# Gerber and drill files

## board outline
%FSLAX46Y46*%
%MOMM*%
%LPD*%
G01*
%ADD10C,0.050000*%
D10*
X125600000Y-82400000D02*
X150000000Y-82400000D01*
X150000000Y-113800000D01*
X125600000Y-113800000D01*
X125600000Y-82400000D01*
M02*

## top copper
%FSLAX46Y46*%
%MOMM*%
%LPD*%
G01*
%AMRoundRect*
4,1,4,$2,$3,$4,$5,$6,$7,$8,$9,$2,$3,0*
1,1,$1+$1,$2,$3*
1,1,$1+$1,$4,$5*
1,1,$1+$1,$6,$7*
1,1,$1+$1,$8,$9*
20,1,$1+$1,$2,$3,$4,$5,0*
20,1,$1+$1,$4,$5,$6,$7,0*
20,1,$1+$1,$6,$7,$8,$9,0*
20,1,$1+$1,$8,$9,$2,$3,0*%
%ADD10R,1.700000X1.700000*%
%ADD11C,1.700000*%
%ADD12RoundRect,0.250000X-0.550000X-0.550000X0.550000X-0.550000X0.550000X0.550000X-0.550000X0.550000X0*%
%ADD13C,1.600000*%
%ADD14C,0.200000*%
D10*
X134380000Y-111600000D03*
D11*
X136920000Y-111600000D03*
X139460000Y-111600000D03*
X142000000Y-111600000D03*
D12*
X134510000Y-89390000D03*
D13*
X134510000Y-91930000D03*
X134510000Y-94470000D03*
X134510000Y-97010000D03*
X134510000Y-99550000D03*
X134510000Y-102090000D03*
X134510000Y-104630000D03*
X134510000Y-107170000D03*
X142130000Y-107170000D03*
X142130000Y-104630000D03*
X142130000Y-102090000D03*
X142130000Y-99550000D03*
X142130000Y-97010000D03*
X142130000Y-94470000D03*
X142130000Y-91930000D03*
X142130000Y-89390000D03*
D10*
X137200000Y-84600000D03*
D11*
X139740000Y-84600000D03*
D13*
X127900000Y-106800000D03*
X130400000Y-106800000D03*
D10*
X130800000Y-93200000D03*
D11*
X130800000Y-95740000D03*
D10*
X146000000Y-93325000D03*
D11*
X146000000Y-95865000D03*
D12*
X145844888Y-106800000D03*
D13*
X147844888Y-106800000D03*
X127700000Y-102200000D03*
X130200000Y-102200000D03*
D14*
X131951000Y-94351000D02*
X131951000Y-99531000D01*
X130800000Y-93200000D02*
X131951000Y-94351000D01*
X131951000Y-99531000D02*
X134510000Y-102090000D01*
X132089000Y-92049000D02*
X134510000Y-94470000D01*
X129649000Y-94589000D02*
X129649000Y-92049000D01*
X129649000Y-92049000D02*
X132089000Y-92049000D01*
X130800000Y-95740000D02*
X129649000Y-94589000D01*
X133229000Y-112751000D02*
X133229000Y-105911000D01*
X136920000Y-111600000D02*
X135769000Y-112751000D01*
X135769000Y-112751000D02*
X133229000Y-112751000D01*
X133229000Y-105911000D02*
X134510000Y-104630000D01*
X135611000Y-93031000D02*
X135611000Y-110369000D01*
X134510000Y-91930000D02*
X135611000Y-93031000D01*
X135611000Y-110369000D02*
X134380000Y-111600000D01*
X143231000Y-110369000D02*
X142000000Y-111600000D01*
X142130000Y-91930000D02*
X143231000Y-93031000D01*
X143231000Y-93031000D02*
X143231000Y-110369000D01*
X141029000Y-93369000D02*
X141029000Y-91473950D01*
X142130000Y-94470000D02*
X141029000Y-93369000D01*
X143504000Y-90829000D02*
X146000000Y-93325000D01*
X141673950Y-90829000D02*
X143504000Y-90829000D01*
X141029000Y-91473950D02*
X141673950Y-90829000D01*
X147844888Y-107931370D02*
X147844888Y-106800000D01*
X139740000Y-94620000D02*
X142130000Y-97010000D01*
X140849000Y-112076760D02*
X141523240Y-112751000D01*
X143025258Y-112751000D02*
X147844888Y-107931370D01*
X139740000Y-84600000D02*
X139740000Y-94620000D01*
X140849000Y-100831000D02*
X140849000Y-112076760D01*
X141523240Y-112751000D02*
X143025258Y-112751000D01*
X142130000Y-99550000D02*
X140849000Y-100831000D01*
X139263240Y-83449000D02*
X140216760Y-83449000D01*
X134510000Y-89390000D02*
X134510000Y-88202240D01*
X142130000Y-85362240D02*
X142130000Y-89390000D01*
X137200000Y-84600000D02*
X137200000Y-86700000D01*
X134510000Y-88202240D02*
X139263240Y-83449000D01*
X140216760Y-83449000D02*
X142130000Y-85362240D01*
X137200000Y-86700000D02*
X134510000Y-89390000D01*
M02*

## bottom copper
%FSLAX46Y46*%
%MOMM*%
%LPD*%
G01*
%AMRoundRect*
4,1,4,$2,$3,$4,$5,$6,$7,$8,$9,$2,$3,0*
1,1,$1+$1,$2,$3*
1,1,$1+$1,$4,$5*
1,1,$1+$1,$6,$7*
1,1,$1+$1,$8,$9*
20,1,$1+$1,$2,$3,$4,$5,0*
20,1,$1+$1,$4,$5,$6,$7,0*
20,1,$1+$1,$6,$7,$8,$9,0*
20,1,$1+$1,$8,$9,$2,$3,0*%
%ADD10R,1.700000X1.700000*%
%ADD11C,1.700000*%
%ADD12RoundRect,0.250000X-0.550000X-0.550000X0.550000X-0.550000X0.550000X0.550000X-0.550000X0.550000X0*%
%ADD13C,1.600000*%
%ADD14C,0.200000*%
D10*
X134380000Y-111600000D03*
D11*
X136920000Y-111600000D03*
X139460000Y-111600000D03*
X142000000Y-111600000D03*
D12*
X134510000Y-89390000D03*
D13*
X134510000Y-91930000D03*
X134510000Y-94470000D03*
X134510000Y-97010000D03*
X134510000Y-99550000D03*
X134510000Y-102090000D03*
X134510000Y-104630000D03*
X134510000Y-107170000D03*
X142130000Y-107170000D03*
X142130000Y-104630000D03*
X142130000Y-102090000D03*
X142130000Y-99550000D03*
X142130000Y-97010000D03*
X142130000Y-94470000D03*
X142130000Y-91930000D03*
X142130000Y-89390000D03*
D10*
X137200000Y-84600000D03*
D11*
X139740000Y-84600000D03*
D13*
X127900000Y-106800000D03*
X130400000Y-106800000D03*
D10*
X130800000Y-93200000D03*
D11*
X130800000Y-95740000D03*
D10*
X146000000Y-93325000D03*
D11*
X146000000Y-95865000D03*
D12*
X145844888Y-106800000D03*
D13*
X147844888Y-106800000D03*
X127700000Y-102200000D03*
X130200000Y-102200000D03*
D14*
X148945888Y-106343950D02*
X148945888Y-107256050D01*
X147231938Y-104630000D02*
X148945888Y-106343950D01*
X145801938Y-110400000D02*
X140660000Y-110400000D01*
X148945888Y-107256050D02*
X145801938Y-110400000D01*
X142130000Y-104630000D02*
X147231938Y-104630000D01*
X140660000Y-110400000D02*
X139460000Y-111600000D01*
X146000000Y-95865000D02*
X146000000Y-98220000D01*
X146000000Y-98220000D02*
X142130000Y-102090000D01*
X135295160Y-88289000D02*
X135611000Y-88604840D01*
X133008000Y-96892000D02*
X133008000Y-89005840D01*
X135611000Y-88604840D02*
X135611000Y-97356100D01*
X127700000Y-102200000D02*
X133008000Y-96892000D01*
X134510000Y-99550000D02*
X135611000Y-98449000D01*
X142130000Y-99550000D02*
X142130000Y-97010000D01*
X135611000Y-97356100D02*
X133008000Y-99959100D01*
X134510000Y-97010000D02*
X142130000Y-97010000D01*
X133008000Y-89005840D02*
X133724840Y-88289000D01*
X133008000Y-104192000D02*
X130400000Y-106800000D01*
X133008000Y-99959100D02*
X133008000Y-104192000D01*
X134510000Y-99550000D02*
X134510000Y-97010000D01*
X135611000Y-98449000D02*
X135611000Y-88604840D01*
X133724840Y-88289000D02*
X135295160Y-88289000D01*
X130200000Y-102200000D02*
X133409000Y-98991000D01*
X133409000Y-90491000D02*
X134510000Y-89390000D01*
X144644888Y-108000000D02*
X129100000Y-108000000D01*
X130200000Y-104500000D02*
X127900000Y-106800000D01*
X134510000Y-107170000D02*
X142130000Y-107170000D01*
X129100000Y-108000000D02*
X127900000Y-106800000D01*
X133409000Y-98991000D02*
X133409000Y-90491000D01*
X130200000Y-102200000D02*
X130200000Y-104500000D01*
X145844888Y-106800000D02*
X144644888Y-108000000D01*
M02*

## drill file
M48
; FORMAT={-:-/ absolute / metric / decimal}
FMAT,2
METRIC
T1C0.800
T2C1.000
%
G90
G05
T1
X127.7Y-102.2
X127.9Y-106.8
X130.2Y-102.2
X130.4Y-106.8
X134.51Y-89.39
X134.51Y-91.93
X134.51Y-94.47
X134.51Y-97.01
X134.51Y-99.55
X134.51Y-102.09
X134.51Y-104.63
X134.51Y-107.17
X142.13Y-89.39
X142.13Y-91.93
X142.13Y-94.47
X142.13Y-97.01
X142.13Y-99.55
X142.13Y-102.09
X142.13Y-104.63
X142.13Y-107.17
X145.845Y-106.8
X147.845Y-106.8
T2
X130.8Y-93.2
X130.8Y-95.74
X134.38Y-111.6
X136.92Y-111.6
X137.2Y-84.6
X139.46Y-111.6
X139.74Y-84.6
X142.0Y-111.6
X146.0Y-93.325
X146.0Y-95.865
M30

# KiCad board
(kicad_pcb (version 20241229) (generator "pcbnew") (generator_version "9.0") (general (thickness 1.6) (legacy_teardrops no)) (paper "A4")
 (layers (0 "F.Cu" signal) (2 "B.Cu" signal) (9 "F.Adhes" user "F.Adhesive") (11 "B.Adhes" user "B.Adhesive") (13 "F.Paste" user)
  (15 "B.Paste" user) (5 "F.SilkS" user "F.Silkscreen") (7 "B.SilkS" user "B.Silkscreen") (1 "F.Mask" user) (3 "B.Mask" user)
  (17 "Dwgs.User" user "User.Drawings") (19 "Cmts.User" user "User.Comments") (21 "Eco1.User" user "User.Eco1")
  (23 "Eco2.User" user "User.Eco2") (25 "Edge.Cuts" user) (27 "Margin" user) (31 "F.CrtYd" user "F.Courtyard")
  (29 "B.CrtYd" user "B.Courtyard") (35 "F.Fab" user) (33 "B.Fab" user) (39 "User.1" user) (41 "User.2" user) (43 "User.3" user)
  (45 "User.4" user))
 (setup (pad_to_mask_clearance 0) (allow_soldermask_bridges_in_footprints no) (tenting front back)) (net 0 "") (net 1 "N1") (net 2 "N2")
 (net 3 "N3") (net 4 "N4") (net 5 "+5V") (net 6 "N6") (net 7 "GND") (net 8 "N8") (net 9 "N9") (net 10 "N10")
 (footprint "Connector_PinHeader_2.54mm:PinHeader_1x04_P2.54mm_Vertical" (layer "F.Cu") (at 134.38 111.6 90)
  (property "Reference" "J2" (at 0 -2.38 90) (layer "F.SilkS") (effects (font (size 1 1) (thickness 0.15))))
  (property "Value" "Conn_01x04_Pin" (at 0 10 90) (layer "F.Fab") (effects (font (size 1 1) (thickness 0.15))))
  (pad "1" thru_hole rect (at 0 0 90) (size 1.7 1.7) (drill 1) (layers "*.Cu" "*.Mask") (remove_unused_layers no) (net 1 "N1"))
  (pad "2" thru_hole circle (at 0 2.54 90) (size 1.7 1.7) (drill 1) (layers "*.Cu" "*.Mask") (remove_unused_layers no) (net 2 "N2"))
  (pad "3" thru_hole circle (at 0 5.08 90) (size 1.7 1.7) (drill 1) (layers "*.Cu" "*.Mask") (remove_unused_layers no) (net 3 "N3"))
  (pad "4" thru_hole circle (at 0 7.62 90) (size 1.7 1.7) (drill 1) (layers "*.Cu" "*.Mask") (remove_unused_layers no) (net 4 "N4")))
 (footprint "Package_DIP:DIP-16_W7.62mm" (layer "F.Cu") (at 134.51 89.39)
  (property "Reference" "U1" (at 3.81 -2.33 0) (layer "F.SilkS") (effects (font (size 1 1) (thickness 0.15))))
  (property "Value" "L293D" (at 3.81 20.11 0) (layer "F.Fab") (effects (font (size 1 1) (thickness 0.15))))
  (pad "1" thru_hole roundrect (at 0 0) (size 1.6 1.6) (drill 0.8) (layers "*.Cu" "*.Mask") (remove_unused_layers no)
   (roundrect_rratio 0.15625) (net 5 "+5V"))
  (pad "2" thru_hole circle (at 0 2.54) (size 1.6 1.6) (drill 0.8) (layers "*.Cu" "*.Mask") (remove_unused_layers no) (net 1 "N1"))
  (pad "3" thru_hole circle (at 0 5.08) (size 1.6 1.6) (drill 0.8) (layers "*.Cu" "*.Mask") (remove_unused_layers no) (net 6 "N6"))
  (pad "4" thru_hole circle (at 0 7.62) (size 1.6 1.6) (drill 0.8) (layers "*.Cu" "*.Mask") (remove_unused_layers no) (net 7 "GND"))
  (pad "5" thru_hole circle (at 0 10.16) (size 1.6 1.6) (drill 0.8) (layers "*.Cu" "*.Mask") (remove_unused_layers no) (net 7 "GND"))
  (pad "6" thru_hole circle (at 0 12.7) (size 1.6 1.6) (drill 0.8) (layers "*.Cu" "*.Mask") (remove_unused_layers no) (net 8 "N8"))
  (pad "7" thru_hole circle (at 0 15.24) (size 1.6 1.6) (drill 0.8) (layers "*.Cu" "*.Mask") (remove_unused_layers no) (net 2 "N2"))
  (pad "8" thru_hole circle (at 0 17.78) (size 1.6 1.6) (drill 0.8) (layers "*.Cu" "*.Mask") (remove_unused_layers no) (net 5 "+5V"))
  (pad "9" thru_hole circle (at 7.62 17.78) (size 1.6 1.6) (drill 0.8) (layers "*.Cu" "*.Mask") (remove_unused_layers no) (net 5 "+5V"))
  (pad "10" thru_hole circle (at 7.62 15.24) (size 1.6 1.6) (drill 0.8) (layers "*.Cu" "*.Mask") (remove_unused_layers no) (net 3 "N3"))
  (pad "11" thru_hole circle (at 7.62 12.7) (size 1.6 1.6) (drill 0.8) (layers "*.Cu" "*.Mask") (remove_unused_layers no) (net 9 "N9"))
  (pad "12" thru_hole circle (at 7.62 10.16) (size 1.6 1.6) (drill 0.8) (layers "*.Cu" "*.Mask") (remove_unused_layers no) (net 7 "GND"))
  (pad "13" thru_hole circle (at 7.62 7.62) (size 1.6 1.6) (drill 0.8) (layers "*.Cu" "*.Mask") (remove_unused_layers no) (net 7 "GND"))
  (pad "14" thru_hole circle (at 7.62 5.08) (size 1.6 1.6) (drill 0.8) (layers "*.Cu" "*.Mask") (remove_unused_layers no) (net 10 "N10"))
  (pad "15" thru_hole circle (at 7.62 2.54) (size 1.6 1.6) (drill 0.8) (layers "*.Cu" "*.Mask") (remove_unused_layers no) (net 4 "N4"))
  (pad "16" thru_hole circle (at 7.62 0) (size 1.6 1.6) (drill 0.8) (layers "*.Cu" "*.Mask") (remove_unused_layers no) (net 5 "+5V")))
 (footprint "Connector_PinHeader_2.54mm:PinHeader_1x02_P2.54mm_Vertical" (layer "F.Cu") (at 137.2 84.6 90)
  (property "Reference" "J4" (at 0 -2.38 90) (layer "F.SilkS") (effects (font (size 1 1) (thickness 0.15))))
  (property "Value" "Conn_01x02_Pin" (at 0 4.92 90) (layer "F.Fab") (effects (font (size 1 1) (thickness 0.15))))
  (pad "1" thru_hole rect (at 0 0 90) (size 1.7 1.7) (drill 1) (layers "*.Cu" "*.Mask") (remove_unused_layers no) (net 5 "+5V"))
  (pad "2" thru_hole circle (at 0 2.54 90) (size 1.7 1.7) (drill 1) (layers "*.Cu" "*.Mask") (remove_unused_layers no) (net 7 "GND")))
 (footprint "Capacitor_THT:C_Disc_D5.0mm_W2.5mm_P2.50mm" (layer "F.Cu") (at 127.9 106.8)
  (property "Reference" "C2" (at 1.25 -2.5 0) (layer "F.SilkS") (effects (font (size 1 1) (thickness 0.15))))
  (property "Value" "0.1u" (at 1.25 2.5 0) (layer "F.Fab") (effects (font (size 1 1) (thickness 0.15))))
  (pad "1" thru_hole circle (at 0 0) (size 1.6 1.6) (drill 0.8) (layers "*.Cu" "*.Mask") (remove_unused_layers no) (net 5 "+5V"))
  (pad "2" thru_hole circle (at 2.5 0) (size 1.6 1.6) (drill 0.8) (layers "*.Cu" "*.Mask") (remove_unused_layers no) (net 7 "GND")))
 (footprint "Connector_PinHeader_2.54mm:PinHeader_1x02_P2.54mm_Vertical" (layer "F.Cu") (at 130.8 93.2)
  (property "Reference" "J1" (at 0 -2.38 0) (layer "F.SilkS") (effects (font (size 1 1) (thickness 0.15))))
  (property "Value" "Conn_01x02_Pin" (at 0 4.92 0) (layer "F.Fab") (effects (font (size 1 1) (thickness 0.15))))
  (pad "1" thru_hole rect (at 0 0) (size 1.7 1.7) (drill 1) (layers "*.Cu" "*.Mask") (remove_unused_layers no) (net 8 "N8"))
  (pad "2" thru_hole circle (at 0 2.54) (size 1.7 1.7) (drill 1) (layers "*.Cu" "*.Mask") (remove_unused_layers no) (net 6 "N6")))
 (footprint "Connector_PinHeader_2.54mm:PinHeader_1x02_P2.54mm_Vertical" (layer "F.Cu") (at 146 93.325)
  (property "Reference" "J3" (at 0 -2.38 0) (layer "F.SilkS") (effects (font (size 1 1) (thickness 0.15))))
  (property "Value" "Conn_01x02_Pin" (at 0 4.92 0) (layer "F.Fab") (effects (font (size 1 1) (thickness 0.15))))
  (pad "1" thru_hole rect (at 0 0) (size 1.7 1.7) (drill 1) (layers "*.Cu" "*.Mask") (remove_unused_layers no) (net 10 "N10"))
  (pad "2" thru_hole circle (at 0 2.54) (size 1.7 1.7) (drill 1) (layers "*.Cu" "*.Mask") (remove_unused_layers no) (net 9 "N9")))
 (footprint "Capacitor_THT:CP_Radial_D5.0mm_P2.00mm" (layer "F.Cu") (at 145.844888 106.8)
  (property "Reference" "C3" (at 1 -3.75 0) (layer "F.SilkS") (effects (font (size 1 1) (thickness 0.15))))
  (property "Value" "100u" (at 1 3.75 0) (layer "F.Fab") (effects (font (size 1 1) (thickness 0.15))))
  (pad "1" thru_hole roundrect (at 0 0) (size 1.6 1.6) (drill 0.8) (layers "*.Cu" "*.Mask") (remove_unused_layers no)
   (roundrect_rratio 0.15625) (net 5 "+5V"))
  (pad "2" thru_hole circle (at 2 0) (size 1.6 1.6) (drill 0.8) (layers "*.Cu" "*.Mask") (remove_unused_layers no) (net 7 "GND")))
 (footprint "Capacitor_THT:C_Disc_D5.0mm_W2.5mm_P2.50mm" (layer "F.Cu") (at 127.7 102.2)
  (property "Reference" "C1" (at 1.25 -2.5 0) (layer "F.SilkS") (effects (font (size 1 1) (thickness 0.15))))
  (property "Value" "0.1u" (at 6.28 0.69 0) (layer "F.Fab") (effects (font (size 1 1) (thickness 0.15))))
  (pad "1" thru_hole circle (at 0 0) (size 1.6 1.6) (drill 0.8) (layers "*.Cu" "*.Mask") (remove_unused_layers no) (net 7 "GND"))
  (pad "2" thru_hole circle (at 2.5 0) (size 1.6 1.6) (drill 0.8) (layers "*.Cu" "*.Mask") (remove_unused_layers no) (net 5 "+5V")))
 (gr_rect (start 125.6 82.4) (end 150 113.8) (stroke (width 0.05) (type default)) (fill no) (layer "Edge.Cuts"))
 (segment (start 131.951 94.351) (end 131.951 99.531) (width 0.2) (layer "F.Cu") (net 8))
 (segment (start 130.8 93.2) (end 131.951 94.351) (width 0.2) (layer "F.Cu") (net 8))
 (segment (start 131.951 99.531) (end 134.51 102.09) (width 0.2) (layer "F.Cu") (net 8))
 (segment (start 132.089 92.049) (end 134.51 94.47) (width 0.2) (layer "F.Cu") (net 6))
 (segment (start 129.649 94.589) (end 129.649 92.049) (width 0.2) (layer "F.Cu") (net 6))
 (segment (start 129.649 92.049) (end 132.089 92.049) (width 0.2) (layer "F.Cu") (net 6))
 (segment (start 130.8 95.74) (end 129.649 94.589) (width 0.2) (layer "F.Cu") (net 6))
 (segment (start 133.229 112.751) (end 133.229 105.911) (width 0.2) (layer "F.Cu") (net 2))
 (segment (start 136.92 111.6) (end 135.769 112.751) (width 0.2) (layer "F.Cu") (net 2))
 (segment (start 135.769 112.751) (end 133.229 112.751) (width 0.2) (layer "F.Cu") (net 2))
 (segment (start 133.229 105.911) (end 134.51 104.63) (width 0.2) (layer "F.Cu") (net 2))
 (segment (start 135.611 93.031) (end 135.611 110.369) (width 0.2) (layer "F.Cu") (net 1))
 (segment (start 134.51 91.93) (end 135.611 93.031) (width 0.2) (layer "F.Cu") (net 1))
 (segment (start 135.611 110.369) (end 134.38 111.6) (width 0.2) (layer "F.Cu") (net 1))
 (segment (start 143.231 110.369) (end 142 111.6) (width 0.2) (layer "F.Cu") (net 4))
 (segment (start 142.13 91.93) (end 143.231 93.031) (width 0.2) (layer "F.Cu") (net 4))
 (segment (start 143.231 93.031) (end 143.231 110.369) (width 0.2) (layer "F.Cu") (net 4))
 (segment (start 148.945888 106.34395) (end 148.945888 107.25605) (width 0.2) (layer "B.Cu") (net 3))
 (segment (start 147.231938 104.63) (end 148.945888 106.34395) (width 0.2) (layer "B.Cu") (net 3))
 (segment (start 145.801938 110.4) (end 140.66 110.4) (width 0.2) (layer "B.Cu") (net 3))
 (segment (start 148.945888 107.25605) (end 145.801938 110.4) (width 0.2) (layer "B.Cu") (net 3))
 (segment (start 142.13 104.63) (end 147.231938 104.63) (width 0.2) (layer "B.Cu") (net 3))
 (segment (start 140.66 110.4) (end 139.46 111.6) (width 0.2) (layer "B.Cu") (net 3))
 (segment (start 146 95.865) (end 146 98.22) (width 0.2) (layer "B.Cu") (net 9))
 (segment (start 146 98.22) (end 142.13 102.09) (width 0.2) (layer "B.Cu") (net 9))
 (segment (start 141.029 93.369) (end 141.029 91.47395) (width 0.2) (layer "F.Cu") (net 10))
 (segment (start 142.13 94.47) (end 141.029 93.369) (width 0.2) (layer "F.Cu") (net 10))
 (segment (start 143.504 90.829) (end 146 93.325) (width 0.2) (layer "F.Cu") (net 10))
 (segment (start 141.67395 90.829) (end 143.504 90.829) (width 0.2) (layer "F.Cu") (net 10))
 (segment (start 141.029 91.47395) (end 141.67395 90.829) (width 0.2) (layer "F.Cu") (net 10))
 (segment (start 147.844888 107.93137) (end 147.844888 106.8) (width 0.2) (layer "F.Cu") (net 7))
 (segment (start 139.74 94.62) (end 142.13 97.01) (width 0.2) (layer "F.Cu") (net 7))
 (segment (start 140.849 112.07676) (end 141.52324 112.751) (width 0.2) (layer "F.Cu") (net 7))
 (segment (start 143.025258 112.751) (end 147.844888 107.93137) (width 0.2) (layer "F.Cu") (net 7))
 (segment (start 139.74 84.6) (end 139.74 94.62) (width 0.2) (layer "F.Cu") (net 7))
 (segment (start 140.849 100.831) (end 140.849 112.07676) (width 0.2) (layer "F.Cu") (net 7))
 (segment (start 141.52324 112.751) (end 143.025258 112.751) (width 0.2) (layer "F.Cu") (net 7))
 (segment (start 142.13 99.55) (end 140.849 100.831) (width 0.2) (layer "F.Cu") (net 7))
 (segment (start 135.29516 88.289) (end 135.611 88.60484) (width 0.2) (layer "B.Cu") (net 7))
 (segment (start 133.008 96.892) (end 133.008 89.00584) (width 0.2) (layer "B.Cu") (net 7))
 (segment (start 135.611 88.60484) (end 135.611 97.3561) (width 0.2) (layer "B.Cu") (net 7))
 (segment (start 127.7 102.2) (end 133.008 96.892) (width 0.2) (layer "B.Cu") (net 7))
 (segment (start 134.51 99.55) (end 135.611 98.449) (width 0.2) (layer "B.Cu") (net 7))
 (segment (start 142.13 99.55) (end 142.13 97.01) (width 0.2) (layer "B.Cu") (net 7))
 (segment (start 135.611 97.3561) (end 133.008 99.9591) (width 0.2) (layer "B.Cu") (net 7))
 (segment (start 134.51 97.01) (end 142.13 97.01) (width 0.2) (layer "B.Cu") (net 7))
 (segment (start 133.008 89.00584) (end 133.72484 88.289) (width 0.2) (layer "B.Cu") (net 7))
 (segment (start 133.008 104.192) (end 130.4 106.8) (width 0.2) (layer "B.Cu") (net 7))
 (segment (start 133.008 99.9591) (end 133.008 104.192) (width 0.2) (layer "B.Cu") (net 7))
 (segment (start 134.51 99.55) (end 134.51 97.01) (width 0.2) (layer "B.Cu") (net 7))
 (segment (start 135.611 98.449) (end 135.611 88.60484) (width 0.2) (layer "B.Cu") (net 7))
 (segment (start 133.72484 88.289) (end 135.29516 88.289) (width 0.2) (layer "B.Cu") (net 7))
 (segment (start 139.26324 83.449) (end 140.21676 83.449) (width 0.2) (layer "F.Cu") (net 5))
 (segment (start 134.51 89.39) (end 134.51 88.20224) (width 0.2) (layer "F.Cu") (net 5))
 (segment (start 142.13 85.36224) (end 142.13 89.39) (width 0.2) (layer "F.Cu") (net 5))
 (segment (start 137.2 84.6) (end 137.2 86.7) (width 0.2) (layer "F.Cu") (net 5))
 (segment (start 134.51 88.20224) (end 139.26324 83.449) (width 0.2) (layer "F.Cu") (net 5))
 (segment (start 140.21676 83.449) (end 142.13 85.36224) (width 0.2) (layer "F.Cu") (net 5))
 (segment (start 137.2 86.7) (end 134.51 89.39) (width 0.2) (layer "F.Cu") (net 5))
 (segment (start 130.2 102.2) (end 133.409 98.991) (width 0.2) (layer "B.Cu") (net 5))
 (segment (start 133.409 90.491) (end 134.51 89.39) (width 0.2) (layer "B.Cu") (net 5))
 (segment (start 144.644888 108) (end 129.1 108) (width 0.2) (layer "B.Cu") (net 5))
 (segment (start 130.2 104.5) (end 127.9 106.8) (width 0.2) (layer "B.Cu") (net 5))
 (segment (start 134.51 107.17) (end 142.13 107.17) (width 0.2) (layer "B.Cu") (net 5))
 (segment (start 129.1 108) (end 127.9 106.8) (width 0.2) (layer "B.Cu") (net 5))
 (segment (start 133.409 98.991) (end 133.409 90.491) (width 0.2) (layer "B.Cu") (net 5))
 (segment (start 130.2 102.2) (end 130.2 104.5) (width 0.2) (layer "B.Cu") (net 5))
 (segment (start 145.844888 106.8) (end 144.644888 108) (width 0.2) (layer "B.Cu") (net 5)))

